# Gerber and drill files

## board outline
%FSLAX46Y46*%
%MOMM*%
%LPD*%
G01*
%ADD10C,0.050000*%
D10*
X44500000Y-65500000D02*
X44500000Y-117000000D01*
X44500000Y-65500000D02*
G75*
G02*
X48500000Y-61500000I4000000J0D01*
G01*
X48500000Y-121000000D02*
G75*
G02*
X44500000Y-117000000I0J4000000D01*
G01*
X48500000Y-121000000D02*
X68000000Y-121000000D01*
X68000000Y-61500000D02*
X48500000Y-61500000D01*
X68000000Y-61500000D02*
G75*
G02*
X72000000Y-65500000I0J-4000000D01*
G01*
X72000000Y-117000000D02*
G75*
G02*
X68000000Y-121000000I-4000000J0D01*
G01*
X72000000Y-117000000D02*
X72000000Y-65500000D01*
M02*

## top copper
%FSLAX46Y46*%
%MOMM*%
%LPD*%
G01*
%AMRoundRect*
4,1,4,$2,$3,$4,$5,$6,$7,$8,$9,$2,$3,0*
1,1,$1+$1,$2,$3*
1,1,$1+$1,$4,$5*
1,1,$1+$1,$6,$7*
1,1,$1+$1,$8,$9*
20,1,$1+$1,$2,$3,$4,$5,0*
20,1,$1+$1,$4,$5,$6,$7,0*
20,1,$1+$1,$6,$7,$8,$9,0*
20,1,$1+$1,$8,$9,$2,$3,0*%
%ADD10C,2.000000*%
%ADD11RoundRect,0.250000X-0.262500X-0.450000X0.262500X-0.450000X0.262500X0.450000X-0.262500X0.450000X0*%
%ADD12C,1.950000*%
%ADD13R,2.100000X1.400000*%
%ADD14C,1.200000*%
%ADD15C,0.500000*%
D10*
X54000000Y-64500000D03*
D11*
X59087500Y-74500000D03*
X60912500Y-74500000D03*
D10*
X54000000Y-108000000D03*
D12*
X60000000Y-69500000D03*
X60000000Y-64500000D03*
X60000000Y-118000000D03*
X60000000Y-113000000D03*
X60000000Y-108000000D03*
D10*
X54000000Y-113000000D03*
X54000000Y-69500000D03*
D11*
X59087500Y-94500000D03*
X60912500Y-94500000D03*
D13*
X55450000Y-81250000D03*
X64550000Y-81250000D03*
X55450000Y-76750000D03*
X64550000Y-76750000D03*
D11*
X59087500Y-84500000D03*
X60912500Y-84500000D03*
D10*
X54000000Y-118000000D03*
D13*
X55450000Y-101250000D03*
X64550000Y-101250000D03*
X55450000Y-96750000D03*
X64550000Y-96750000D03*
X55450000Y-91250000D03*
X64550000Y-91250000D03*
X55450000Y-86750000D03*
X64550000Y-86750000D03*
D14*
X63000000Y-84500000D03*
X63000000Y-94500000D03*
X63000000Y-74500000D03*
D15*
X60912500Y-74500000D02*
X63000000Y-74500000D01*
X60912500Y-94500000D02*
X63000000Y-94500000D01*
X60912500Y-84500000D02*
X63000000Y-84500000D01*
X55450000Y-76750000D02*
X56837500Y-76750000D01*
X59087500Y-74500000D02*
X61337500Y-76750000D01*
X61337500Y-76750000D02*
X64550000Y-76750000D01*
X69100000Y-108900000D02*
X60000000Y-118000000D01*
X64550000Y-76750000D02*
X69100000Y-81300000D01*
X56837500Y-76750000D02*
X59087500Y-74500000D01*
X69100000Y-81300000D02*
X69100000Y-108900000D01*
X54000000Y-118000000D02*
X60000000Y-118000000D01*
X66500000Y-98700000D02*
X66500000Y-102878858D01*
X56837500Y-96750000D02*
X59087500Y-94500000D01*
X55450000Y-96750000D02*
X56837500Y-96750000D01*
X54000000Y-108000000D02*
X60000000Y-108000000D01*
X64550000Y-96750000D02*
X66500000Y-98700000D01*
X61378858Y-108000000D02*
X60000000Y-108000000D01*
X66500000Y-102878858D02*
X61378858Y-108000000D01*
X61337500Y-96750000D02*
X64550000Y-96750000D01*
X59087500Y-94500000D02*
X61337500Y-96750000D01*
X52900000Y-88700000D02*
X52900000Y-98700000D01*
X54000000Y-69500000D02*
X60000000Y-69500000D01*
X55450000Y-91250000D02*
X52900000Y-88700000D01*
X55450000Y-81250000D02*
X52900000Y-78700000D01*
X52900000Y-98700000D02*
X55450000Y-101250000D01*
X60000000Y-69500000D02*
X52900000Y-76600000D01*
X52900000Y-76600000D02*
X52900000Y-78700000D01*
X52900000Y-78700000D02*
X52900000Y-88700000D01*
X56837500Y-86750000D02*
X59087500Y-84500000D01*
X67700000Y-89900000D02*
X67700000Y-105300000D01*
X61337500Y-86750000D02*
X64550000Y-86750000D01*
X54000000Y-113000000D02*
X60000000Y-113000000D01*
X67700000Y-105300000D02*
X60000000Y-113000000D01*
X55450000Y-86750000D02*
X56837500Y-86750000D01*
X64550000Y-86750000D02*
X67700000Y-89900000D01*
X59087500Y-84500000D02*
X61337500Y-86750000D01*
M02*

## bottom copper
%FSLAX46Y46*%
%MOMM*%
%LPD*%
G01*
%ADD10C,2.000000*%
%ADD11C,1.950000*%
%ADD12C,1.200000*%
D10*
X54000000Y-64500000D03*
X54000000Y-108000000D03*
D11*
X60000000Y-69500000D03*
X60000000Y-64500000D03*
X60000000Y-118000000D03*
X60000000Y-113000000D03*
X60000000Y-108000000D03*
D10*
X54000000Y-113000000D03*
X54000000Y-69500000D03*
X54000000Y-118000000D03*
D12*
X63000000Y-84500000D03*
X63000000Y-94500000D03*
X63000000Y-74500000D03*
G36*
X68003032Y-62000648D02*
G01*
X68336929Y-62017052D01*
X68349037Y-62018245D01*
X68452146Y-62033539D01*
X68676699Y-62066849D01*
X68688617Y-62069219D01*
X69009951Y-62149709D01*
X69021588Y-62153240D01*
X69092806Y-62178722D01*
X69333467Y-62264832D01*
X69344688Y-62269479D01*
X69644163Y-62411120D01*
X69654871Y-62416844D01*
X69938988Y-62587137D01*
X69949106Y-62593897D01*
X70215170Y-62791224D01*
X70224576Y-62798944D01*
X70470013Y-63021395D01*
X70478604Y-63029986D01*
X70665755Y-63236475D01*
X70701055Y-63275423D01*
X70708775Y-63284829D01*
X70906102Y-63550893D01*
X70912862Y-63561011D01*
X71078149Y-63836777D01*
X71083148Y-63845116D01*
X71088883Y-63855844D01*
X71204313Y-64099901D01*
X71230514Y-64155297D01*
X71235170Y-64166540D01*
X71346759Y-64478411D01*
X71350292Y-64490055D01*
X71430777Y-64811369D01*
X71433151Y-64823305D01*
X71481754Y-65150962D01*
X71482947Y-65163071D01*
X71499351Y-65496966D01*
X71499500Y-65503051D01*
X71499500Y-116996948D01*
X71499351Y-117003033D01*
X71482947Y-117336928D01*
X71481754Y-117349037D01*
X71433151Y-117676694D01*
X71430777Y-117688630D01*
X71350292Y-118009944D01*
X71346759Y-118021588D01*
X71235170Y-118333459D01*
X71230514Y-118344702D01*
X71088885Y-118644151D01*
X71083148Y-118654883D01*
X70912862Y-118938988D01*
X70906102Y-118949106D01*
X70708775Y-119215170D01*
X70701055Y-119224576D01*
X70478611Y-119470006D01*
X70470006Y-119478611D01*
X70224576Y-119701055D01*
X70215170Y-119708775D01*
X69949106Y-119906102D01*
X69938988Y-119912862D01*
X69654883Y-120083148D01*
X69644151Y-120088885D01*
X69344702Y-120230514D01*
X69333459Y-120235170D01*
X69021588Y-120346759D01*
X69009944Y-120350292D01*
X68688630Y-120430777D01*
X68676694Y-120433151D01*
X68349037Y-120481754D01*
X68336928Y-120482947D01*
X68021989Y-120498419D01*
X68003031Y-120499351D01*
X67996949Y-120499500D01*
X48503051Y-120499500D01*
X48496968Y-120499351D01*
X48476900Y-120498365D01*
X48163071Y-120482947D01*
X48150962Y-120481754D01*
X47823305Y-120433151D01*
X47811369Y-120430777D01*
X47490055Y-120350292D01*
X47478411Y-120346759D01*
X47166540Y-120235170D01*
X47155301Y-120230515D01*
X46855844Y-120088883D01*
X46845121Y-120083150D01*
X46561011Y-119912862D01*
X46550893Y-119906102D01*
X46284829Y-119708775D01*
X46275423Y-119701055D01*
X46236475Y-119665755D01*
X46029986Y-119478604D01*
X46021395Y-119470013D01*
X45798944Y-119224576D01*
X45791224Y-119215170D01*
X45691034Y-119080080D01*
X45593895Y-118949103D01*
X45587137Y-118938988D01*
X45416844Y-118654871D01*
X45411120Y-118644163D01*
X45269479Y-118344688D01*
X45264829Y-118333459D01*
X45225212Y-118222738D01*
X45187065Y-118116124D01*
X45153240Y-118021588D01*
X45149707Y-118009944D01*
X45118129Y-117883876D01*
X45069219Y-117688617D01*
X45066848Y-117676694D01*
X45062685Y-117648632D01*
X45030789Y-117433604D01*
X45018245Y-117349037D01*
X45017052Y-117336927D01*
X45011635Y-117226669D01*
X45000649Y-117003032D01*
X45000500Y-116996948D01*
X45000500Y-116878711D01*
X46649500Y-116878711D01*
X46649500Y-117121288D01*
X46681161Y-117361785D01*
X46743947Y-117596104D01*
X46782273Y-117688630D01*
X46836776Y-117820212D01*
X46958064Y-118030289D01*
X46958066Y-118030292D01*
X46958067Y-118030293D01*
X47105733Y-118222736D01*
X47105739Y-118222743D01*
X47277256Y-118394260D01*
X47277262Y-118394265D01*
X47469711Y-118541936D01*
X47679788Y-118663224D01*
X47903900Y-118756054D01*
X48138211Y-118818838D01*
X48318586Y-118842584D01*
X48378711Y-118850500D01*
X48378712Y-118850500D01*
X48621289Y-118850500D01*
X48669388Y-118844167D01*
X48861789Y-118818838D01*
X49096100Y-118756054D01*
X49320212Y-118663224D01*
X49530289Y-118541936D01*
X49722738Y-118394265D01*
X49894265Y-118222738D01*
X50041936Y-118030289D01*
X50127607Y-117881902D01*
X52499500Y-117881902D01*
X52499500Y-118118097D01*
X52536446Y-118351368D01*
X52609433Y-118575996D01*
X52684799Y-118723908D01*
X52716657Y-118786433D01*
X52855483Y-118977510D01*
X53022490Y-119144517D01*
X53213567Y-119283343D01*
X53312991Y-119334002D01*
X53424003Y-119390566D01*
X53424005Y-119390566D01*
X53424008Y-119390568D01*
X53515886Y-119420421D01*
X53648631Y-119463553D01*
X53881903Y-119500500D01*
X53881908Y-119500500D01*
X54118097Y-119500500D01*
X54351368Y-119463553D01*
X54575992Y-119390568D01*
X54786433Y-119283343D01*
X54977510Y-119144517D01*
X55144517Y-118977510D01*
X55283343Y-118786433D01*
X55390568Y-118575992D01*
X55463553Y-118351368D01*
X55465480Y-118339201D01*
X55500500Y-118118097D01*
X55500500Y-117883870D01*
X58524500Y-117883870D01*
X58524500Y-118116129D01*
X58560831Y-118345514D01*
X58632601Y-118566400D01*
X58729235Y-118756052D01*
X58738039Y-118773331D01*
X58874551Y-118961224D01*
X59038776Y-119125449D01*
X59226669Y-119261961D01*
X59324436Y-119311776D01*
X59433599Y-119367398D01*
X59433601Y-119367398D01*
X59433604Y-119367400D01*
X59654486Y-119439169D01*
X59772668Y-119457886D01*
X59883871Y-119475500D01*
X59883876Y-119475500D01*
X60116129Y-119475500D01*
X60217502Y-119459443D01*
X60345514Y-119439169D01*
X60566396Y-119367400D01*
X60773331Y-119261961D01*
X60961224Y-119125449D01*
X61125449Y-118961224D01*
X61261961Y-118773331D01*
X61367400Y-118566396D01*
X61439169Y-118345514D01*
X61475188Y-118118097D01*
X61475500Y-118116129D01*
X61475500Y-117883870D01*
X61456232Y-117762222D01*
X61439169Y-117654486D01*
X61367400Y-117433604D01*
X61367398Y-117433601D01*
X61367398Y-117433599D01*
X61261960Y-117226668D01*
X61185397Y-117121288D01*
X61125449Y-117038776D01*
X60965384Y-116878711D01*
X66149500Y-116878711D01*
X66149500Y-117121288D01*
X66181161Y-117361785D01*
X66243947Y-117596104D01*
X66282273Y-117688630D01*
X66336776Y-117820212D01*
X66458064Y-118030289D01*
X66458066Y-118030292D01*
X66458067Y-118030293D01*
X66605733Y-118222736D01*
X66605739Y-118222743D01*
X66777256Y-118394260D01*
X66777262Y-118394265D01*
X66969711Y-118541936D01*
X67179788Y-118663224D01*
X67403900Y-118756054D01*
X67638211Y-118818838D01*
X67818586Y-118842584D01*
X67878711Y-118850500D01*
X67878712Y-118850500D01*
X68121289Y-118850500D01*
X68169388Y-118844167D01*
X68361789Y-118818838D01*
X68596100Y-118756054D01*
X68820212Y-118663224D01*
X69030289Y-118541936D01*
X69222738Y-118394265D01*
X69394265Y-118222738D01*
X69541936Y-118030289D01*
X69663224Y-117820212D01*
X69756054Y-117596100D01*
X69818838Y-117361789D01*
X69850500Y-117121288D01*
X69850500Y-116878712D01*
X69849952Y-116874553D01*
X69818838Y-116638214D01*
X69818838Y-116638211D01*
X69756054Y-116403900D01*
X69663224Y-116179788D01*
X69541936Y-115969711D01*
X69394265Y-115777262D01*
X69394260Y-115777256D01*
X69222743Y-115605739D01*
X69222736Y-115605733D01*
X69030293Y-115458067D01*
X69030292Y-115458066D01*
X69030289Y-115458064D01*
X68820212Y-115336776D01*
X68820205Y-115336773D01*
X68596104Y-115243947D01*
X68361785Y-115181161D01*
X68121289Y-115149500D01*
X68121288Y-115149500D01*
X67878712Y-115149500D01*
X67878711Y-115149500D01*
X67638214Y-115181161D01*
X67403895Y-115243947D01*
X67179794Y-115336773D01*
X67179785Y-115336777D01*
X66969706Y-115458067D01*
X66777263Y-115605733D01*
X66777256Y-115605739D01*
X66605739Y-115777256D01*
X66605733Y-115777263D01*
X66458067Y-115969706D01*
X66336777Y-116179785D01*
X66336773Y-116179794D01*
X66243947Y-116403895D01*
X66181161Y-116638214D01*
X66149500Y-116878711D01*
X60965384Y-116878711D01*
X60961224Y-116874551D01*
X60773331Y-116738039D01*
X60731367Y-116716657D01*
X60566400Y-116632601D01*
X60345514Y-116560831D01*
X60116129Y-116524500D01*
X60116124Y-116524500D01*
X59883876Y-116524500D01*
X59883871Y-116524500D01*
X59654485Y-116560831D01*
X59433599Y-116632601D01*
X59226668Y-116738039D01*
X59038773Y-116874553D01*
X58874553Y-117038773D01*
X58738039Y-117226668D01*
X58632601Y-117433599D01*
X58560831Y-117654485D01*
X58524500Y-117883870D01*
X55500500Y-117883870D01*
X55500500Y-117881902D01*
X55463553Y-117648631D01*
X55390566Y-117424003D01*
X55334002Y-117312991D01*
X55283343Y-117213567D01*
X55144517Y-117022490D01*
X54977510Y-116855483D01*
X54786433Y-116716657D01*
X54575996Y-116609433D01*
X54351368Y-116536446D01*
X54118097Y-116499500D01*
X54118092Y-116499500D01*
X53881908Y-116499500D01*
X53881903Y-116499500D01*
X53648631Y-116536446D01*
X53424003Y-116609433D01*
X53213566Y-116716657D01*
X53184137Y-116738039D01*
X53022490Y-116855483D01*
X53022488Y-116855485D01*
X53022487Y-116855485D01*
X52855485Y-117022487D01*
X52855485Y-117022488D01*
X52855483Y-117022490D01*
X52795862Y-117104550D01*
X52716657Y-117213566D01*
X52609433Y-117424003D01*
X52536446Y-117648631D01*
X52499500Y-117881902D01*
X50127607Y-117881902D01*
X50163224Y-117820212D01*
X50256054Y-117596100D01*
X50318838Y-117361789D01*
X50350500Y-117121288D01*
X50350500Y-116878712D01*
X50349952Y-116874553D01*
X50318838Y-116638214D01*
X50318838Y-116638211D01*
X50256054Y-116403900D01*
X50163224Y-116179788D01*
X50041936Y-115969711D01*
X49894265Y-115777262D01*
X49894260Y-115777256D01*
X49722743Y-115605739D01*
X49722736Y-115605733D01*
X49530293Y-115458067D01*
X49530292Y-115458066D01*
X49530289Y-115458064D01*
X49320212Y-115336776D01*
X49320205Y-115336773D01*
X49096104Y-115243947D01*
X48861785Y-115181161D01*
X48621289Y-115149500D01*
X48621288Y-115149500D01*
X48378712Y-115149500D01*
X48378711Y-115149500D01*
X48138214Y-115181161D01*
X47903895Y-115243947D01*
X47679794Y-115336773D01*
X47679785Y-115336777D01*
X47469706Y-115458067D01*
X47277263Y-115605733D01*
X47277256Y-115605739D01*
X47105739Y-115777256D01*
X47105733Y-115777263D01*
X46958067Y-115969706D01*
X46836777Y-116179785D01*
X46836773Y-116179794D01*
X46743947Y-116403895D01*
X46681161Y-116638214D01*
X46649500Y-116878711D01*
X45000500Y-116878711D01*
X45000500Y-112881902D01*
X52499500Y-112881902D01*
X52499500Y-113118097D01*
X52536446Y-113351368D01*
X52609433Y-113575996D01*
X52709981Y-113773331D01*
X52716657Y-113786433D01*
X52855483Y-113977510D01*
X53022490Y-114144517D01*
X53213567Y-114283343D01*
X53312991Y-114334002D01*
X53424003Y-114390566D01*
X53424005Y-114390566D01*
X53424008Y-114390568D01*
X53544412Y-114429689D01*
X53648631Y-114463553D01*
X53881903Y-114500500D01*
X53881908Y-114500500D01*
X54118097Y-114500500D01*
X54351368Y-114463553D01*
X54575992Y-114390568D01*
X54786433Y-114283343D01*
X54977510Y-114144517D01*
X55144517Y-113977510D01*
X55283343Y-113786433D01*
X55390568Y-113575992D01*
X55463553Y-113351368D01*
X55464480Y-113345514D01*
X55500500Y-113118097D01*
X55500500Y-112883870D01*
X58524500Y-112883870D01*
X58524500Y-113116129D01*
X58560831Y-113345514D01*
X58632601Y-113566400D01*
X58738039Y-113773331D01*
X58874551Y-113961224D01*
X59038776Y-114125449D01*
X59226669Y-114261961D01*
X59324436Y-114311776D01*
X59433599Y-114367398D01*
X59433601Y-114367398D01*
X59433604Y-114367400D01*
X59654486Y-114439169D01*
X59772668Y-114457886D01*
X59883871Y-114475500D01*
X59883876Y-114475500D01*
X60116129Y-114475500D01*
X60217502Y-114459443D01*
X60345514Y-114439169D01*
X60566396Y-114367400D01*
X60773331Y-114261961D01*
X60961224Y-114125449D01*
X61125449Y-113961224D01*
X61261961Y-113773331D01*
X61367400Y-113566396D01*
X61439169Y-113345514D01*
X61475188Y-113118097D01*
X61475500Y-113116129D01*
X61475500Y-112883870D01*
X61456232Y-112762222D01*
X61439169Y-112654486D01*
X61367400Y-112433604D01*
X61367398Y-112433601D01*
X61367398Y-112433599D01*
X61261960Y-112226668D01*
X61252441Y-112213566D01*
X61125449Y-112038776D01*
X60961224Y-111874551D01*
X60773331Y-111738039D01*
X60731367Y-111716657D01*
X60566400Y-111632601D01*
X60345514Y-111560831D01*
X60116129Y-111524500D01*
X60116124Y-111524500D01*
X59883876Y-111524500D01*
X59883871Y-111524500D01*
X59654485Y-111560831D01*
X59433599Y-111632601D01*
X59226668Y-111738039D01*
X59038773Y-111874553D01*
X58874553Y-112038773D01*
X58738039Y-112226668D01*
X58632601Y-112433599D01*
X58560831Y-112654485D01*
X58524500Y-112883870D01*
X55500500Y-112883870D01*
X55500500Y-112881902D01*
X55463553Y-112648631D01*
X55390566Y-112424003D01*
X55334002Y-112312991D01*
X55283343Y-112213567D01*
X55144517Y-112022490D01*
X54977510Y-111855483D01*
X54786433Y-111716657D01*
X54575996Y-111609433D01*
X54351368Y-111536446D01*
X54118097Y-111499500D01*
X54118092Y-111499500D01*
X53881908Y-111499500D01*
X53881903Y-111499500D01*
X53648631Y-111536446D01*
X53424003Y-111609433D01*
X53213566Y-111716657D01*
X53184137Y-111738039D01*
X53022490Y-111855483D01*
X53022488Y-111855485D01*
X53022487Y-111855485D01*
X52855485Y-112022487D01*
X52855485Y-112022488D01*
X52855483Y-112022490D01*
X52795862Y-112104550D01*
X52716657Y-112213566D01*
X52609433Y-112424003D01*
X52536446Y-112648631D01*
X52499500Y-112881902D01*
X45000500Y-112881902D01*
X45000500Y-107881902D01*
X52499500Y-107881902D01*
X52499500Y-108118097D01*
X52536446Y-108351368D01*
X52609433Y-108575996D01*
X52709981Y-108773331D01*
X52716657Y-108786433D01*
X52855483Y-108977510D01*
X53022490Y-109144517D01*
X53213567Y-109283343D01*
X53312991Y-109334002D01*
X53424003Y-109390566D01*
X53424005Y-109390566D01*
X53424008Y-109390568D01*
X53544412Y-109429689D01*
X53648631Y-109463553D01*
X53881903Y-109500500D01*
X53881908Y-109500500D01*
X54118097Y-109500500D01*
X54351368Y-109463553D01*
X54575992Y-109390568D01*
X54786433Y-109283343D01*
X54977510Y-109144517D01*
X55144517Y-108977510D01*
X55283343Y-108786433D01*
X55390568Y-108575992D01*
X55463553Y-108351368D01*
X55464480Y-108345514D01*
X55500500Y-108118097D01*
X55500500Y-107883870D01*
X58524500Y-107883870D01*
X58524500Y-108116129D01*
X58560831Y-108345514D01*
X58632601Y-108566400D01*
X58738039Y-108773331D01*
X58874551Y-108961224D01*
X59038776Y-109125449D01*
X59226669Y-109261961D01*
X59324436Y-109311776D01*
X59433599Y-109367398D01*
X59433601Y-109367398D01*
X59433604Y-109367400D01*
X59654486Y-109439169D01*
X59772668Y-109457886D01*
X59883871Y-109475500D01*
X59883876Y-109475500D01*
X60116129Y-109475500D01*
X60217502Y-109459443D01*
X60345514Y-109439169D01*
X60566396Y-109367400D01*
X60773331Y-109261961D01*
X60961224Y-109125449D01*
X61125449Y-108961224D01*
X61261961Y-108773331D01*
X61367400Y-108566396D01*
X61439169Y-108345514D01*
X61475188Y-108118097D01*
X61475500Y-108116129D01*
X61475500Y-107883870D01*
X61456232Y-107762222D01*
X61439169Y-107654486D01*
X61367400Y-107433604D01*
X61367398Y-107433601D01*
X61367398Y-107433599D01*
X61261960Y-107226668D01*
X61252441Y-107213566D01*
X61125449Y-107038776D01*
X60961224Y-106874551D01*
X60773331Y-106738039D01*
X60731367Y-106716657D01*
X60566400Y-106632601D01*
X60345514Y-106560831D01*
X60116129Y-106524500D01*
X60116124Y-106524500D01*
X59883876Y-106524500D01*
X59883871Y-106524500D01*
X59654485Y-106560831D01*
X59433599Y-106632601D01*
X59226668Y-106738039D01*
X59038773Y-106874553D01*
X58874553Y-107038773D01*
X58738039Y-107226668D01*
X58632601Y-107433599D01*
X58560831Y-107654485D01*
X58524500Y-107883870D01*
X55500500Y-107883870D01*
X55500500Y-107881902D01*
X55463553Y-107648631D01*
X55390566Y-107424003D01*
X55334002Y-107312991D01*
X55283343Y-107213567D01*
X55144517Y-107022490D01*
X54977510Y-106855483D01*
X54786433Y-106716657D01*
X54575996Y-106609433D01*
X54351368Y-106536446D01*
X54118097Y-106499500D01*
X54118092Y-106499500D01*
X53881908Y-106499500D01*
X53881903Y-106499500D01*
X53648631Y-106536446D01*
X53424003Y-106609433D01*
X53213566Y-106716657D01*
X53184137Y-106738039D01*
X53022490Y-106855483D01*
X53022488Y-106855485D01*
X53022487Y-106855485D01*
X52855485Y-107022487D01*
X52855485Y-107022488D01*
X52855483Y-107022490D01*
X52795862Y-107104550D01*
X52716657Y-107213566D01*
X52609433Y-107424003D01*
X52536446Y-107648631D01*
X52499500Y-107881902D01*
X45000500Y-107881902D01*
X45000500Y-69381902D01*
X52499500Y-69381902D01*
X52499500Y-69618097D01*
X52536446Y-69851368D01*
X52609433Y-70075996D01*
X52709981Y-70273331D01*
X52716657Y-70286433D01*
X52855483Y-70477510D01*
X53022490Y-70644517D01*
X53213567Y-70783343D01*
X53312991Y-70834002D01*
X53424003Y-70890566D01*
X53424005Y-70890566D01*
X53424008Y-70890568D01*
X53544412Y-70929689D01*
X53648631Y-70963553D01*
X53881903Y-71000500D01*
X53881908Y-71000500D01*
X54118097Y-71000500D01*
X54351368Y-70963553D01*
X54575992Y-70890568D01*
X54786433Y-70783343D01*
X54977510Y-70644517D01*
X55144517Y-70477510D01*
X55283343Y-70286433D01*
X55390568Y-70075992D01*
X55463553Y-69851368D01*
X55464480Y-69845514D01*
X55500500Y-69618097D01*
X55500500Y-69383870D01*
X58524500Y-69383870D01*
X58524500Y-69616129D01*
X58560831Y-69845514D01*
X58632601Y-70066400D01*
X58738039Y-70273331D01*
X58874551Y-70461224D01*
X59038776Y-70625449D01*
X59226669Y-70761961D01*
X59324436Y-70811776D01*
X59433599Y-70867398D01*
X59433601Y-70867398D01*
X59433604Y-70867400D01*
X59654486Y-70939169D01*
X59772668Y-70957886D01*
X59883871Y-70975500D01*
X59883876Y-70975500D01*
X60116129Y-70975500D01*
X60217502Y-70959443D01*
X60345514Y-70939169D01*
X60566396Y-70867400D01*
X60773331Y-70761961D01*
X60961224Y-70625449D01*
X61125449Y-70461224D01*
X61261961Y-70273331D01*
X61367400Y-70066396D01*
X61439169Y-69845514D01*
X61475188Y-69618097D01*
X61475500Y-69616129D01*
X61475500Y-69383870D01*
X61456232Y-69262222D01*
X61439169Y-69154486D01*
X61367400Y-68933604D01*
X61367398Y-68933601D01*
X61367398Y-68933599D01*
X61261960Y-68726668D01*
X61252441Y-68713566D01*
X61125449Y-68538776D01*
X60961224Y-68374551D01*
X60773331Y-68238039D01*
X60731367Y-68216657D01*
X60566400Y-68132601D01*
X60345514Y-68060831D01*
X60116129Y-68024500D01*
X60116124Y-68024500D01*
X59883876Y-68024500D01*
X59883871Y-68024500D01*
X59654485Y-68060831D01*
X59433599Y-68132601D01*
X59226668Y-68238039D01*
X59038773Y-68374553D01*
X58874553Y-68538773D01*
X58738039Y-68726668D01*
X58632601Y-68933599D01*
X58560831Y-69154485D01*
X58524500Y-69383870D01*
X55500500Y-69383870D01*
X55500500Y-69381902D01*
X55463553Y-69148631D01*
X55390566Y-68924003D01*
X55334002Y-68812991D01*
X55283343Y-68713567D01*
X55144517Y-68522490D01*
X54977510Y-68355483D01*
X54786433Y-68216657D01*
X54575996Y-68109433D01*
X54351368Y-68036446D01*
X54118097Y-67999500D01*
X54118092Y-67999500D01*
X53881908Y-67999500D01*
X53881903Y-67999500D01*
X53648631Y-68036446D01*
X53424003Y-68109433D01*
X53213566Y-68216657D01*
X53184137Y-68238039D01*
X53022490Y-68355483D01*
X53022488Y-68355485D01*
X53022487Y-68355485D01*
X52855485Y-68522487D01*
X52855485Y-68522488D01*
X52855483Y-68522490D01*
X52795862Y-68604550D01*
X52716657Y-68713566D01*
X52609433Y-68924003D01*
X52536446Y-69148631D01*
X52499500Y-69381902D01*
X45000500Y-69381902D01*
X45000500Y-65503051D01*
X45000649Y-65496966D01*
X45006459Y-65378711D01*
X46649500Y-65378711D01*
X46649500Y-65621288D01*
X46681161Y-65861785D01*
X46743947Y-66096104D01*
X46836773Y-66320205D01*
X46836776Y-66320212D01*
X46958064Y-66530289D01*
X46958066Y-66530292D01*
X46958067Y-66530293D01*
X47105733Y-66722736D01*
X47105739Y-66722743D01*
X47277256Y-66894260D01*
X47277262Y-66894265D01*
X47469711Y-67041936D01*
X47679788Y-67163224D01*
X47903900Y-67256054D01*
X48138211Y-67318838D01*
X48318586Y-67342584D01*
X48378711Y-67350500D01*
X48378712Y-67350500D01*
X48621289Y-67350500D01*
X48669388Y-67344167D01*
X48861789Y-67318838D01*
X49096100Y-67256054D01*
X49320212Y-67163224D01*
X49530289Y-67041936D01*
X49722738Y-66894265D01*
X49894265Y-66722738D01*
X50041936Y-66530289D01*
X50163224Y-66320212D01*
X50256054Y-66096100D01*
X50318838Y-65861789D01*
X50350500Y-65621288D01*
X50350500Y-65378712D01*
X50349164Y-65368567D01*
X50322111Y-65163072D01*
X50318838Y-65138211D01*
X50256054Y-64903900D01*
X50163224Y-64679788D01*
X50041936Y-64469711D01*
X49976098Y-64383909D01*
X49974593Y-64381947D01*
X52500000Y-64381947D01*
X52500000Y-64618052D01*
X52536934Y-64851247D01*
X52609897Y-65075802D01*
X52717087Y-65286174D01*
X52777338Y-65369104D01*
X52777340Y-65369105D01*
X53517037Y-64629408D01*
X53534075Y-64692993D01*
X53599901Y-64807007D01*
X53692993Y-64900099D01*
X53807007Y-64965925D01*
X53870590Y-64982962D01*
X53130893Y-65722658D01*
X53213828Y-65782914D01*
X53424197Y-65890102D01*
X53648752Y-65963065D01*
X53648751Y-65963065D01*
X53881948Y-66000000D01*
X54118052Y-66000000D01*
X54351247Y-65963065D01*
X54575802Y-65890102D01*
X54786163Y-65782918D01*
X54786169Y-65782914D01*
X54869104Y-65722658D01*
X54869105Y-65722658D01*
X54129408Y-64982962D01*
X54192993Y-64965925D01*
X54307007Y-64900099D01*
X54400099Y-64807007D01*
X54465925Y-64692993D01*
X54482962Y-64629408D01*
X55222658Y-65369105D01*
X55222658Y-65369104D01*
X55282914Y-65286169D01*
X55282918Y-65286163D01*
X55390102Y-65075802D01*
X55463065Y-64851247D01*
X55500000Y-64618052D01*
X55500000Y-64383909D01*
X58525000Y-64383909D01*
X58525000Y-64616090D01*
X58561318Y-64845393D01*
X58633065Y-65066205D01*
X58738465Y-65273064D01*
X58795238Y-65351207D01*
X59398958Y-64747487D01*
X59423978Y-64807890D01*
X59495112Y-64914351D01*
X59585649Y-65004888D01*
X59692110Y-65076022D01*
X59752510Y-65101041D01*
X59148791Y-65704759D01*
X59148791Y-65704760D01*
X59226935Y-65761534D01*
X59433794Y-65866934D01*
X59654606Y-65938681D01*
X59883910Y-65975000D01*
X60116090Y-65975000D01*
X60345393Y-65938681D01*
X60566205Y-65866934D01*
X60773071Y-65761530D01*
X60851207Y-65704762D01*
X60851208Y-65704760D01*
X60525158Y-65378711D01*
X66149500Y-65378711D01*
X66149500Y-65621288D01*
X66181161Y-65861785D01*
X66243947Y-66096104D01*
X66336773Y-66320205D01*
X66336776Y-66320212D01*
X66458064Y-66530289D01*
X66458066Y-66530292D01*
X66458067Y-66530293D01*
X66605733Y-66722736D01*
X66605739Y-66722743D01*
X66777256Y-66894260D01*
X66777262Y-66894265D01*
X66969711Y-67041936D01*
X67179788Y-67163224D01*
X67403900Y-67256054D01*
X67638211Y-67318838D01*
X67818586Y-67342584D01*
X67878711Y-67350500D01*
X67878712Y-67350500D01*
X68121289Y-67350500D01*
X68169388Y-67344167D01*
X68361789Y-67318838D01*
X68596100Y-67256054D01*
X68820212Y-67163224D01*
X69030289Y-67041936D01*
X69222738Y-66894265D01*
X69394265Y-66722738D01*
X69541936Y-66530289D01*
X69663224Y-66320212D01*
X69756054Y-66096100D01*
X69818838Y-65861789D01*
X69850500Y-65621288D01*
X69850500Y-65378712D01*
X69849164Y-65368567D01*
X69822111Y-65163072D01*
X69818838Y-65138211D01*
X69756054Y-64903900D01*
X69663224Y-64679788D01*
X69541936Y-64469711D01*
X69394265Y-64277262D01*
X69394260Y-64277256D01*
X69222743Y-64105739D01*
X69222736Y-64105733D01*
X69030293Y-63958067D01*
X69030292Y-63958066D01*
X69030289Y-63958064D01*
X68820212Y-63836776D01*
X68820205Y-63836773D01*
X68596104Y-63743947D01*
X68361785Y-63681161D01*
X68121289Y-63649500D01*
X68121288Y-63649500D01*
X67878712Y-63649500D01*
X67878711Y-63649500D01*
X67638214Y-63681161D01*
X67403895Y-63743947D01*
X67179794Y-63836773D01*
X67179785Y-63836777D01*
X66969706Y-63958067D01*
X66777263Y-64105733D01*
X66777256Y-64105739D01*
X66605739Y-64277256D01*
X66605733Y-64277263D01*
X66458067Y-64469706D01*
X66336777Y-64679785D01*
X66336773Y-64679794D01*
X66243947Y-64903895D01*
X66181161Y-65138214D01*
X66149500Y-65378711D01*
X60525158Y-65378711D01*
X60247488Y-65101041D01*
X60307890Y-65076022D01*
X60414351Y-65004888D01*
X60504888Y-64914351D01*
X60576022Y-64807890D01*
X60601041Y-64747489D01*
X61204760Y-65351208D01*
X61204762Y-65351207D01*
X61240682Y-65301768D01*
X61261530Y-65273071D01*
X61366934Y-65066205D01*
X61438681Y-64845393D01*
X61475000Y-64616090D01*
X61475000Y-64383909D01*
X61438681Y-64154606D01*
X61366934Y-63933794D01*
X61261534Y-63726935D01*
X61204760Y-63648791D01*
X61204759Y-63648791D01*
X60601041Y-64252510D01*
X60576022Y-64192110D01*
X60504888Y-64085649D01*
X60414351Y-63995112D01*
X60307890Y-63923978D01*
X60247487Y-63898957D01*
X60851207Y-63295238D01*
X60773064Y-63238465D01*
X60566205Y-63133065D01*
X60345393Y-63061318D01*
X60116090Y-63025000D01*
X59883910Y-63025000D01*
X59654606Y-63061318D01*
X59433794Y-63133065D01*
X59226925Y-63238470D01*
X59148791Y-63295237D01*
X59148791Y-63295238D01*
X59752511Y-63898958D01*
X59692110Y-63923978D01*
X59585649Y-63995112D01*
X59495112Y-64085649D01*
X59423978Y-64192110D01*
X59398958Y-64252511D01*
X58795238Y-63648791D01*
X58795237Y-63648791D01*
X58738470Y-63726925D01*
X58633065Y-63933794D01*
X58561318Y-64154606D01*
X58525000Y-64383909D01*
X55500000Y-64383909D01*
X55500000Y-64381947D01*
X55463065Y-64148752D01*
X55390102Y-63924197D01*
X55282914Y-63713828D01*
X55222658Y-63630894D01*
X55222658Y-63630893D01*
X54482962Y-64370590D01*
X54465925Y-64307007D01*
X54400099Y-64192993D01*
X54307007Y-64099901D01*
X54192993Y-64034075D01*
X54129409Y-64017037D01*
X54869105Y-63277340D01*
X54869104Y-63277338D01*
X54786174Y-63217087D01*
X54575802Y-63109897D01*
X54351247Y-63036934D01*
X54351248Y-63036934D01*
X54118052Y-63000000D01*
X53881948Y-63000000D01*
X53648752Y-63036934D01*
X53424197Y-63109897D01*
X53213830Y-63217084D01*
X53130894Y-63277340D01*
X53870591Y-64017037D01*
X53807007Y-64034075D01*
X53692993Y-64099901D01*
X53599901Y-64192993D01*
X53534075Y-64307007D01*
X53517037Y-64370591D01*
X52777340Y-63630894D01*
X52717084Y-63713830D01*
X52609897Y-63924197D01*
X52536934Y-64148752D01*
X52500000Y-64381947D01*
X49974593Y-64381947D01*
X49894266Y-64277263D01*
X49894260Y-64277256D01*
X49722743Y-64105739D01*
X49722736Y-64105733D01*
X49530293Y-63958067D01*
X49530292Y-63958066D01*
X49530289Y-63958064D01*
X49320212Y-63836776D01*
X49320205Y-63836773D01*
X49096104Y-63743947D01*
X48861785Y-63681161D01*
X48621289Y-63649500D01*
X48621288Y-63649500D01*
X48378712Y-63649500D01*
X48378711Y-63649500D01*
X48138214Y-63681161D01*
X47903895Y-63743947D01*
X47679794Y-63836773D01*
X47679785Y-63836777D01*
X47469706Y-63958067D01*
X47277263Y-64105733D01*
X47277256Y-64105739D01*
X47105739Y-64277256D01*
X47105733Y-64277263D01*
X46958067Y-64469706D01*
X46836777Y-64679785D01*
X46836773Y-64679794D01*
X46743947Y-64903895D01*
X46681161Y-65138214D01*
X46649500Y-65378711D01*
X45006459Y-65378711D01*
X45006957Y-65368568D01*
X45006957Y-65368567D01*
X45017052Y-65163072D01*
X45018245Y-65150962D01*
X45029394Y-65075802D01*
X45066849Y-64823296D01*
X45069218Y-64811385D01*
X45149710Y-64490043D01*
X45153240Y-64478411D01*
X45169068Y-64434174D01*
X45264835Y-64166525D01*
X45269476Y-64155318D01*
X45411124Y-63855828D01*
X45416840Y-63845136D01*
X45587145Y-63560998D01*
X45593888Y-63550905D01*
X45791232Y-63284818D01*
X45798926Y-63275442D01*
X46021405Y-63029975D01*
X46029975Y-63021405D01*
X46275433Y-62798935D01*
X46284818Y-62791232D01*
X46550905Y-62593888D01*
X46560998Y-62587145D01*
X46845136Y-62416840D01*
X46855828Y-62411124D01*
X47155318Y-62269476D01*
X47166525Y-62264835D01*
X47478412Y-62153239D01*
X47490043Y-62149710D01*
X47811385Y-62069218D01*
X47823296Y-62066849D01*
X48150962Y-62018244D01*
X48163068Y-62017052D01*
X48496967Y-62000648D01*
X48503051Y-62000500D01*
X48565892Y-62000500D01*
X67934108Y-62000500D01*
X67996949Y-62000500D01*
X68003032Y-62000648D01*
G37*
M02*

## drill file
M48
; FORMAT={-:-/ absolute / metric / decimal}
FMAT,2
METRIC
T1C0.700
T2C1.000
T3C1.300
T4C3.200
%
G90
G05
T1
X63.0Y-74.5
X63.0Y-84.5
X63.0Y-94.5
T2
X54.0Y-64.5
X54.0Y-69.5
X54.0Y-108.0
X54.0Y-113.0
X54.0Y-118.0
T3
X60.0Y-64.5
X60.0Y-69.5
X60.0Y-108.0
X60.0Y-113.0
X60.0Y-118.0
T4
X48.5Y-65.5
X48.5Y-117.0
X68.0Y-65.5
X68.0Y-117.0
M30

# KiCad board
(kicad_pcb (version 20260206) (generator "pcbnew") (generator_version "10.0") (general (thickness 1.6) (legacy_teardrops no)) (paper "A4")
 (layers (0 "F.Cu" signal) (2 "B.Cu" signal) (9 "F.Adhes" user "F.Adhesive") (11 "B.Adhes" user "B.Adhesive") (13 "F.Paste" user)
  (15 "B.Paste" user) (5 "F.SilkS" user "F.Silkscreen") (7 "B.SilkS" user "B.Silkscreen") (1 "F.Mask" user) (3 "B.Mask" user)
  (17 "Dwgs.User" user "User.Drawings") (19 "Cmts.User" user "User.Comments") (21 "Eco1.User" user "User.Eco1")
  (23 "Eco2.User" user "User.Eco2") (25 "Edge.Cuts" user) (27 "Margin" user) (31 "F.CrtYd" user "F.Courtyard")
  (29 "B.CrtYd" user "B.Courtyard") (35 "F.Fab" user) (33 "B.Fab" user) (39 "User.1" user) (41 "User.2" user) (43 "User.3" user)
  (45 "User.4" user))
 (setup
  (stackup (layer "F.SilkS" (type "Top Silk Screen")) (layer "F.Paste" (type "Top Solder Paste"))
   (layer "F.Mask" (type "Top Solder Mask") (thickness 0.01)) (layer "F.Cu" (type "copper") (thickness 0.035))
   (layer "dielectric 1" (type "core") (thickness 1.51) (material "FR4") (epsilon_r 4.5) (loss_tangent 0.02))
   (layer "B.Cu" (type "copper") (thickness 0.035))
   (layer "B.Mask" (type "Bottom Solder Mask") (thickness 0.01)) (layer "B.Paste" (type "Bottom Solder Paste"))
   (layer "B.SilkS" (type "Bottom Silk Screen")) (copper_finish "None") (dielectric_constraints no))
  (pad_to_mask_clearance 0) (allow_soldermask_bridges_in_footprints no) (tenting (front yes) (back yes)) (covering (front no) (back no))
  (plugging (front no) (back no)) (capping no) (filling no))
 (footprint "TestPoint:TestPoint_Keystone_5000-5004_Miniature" (layer "F.Cu") (at 54 64.5)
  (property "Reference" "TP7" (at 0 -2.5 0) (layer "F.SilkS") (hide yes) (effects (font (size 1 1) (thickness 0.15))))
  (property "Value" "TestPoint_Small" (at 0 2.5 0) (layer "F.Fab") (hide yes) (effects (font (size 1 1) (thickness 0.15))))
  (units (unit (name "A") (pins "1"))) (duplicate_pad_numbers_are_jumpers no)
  (pad "1" thru_hole circle (at 0 0) (size 2 2) (drill 1) (layers "*.Cu" "*.Mask") (remove_unused_layers no) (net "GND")))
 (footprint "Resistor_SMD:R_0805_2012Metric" (layer "F.Cu") (at 60 74.5)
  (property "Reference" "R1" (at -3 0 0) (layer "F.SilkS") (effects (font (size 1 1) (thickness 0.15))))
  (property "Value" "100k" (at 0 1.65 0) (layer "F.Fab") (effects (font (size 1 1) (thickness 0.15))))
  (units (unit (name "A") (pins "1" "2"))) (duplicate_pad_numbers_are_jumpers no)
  (pad "1" smd roundrect (at -0.9125 0) (size 1.025 1.4) (layers "F.Cu" "F.Mask" "F.Paste") (roundrect_rratio 0.243902) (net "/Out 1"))
  (pad "2" smd roundrect (at 0.9125 0) (size 1.025 1.4) (layers "F.Cu" "F.Mask" "F.Paste") (roundrect_rratio 0.243902) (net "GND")))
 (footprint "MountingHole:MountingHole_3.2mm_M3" (layer "F.Cu") (at 68 117)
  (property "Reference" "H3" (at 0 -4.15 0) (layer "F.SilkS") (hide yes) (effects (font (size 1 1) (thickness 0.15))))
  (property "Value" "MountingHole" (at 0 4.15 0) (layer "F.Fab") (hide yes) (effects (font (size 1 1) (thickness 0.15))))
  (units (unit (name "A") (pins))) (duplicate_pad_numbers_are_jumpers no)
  (pad "" np_thru_hole circle (at 0 0) (size 3.2 3.2) (drill 3.2) (layers "*.Cu" "*.Mask")))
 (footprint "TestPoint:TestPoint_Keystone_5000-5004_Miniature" (layer "F.Cu") (at 54 108)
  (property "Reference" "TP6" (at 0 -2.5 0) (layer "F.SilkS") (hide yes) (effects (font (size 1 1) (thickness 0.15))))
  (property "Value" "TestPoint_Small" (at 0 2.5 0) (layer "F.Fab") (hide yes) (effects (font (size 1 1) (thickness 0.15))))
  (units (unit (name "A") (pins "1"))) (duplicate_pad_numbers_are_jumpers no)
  (pad "1" thru_hole circle (at 0 0) (size 2 2) (drill 1) (layers "*.Cu" "*.Mask") (remove_unused_layers no) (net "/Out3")))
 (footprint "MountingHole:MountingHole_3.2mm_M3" (layer "F.Cu") (at 48.5 117)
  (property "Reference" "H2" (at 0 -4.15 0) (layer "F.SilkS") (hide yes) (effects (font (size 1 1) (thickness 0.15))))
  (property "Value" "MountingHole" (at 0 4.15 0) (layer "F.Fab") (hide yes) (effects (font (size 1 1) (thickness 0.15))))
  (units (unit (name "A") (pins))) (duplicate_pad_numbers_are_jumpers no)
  (pad "" np_thru_hole circle (at 0 0) (size 3.2 3.2) (drill 3.2) (layers "*.Cu" "*.Mask")))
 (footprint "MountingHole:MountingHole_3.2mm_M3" (layer "F.Cu") (at 68 65.5)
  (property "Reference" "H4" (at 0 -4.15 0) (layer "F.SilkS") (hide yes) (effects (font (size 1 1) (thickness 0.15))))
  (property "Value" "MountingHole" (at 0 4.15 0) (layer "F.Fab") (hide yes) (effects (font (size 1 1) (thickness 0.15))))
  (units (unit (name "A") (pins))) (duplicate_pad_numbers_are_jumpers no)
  (pad "" np_thru_hole circle (at 0 0) (size 3.2 3.2) (drill 3.2) (layers "*.Cu" "*.Mask")))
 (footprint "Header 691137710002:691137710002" (layer "F.Cu") (at 60 67 90)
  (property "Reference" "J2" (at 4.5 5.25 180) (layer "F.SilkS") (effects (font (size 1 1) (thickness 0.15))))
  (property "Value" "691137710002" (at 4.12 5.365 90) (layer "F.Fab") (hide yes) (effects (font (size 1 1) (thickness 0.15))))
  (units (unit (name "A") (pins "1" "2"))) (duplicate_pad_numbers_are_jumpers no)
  (pad "1" thru_hole circle (at -2.5 0 90) (size 1.95 1.95) (drill 1.3) (layers "*.Cu" "*.Mask") (remove_unused_layers no) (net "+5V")
   (solder_mask_margin 0.102))
  (pad "2" thru_hole circle (at 2.5 0 90) (size 1.95 1.95) (drill 1.3) (layers "*.Cu" "*.Mask") (remove_unused_layers no) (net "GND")
   (solder_mask_margin 0.102)))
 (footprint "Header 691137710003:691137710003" (layer "F.Cu") (at 60 113 90)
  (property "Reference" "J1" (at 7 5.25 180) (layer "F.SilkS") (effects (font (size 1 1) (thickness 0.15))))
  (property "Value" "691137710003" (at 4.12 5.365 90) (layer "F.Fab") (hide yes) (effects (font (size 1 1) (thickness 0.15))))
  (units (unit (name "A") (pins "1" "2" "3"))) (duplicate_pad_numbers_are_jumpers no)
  (pad "1" thru_hole circle (at -5 0 90) (size 1.95 1.95) (drill 1.3) (layers "*.Cu" "*.Mask") (remove_unused_layers no) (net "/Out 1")
   (solder_mask_margin 0.102))
  (pad "2" thru_hole circle (at 0 0 90) (size 1.95 1.95) (drill 1.3) (layers "*.Cu" "*.Mask") (remove_unused_layers no) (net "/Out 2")
   (solder_mask_margin 0.102))
  (pad "3" thru_hole circle (at 5 0 90) (size 1.95 1.95) (drill 1.3) (layers "*.Cu" "*.Mask") (remove_unused_layers no) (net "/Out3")
   (solder_mask_margin 0.102)))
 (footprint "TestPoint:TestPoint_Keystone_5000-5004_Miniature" (layer "F.Cu") (at 54 113)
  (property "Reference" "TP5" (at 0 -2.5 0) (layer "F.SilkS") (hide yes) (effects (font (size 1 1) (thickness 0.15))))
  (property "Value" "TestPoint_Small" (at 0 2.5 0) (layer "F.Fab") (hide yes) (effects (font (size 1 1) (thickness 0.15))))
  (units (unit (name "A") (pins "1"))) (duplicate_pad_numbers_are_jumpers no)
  (pad "1" thru_hole circle (at 0 0) (size 2 2) (drill 1) (layers "*.Cu" "*.Mask") (remove_unused_layers no) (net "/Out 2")))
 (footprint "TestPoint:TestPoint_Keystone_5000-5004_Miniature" (layer "F.Cu") (at 54 69.5)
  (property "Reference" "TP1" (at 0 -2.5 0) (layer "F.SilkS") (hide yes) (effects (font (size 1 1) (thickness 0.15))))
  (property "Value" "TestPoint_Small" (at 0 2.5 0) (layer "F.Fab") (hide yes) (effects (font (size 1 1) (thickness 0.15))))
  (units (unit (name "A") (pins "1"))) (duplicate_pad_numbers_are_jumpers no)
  (pad "1" thru_hole circle (at 0 0) (size 2 2) (drill 1) (layers "*.Cu" "*.Mask") (remove_unused_layers no) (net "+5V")))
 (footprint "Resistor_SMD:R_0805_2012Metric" (layer "F.Cu") (at 60 94.5)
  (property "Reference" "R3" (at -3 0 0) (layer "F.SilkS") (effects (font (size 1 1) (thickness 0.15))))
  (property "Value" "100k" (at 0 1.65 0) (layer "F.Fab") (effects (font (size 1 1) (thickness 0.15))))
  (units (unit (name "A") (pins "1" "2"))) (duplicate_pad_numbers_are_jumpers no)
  (pad "1" smd roundrect (at -0.9125 0) (size 1.025 1.4) (layers "F.Cu" "F.Mask" "F.Paste") (roundrect_rratio 0.243902) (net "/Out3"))
  (pad "2" smd roundrect (at 0.9125 0) (size 1.025 1.4) (layers "F.Cu" "F.Mask" "F.Paste") (roundrect_rratio 0.243902) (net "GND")))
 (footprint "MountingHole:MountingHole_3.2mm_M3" (layer "F.Cu") (at 48.5 65.5)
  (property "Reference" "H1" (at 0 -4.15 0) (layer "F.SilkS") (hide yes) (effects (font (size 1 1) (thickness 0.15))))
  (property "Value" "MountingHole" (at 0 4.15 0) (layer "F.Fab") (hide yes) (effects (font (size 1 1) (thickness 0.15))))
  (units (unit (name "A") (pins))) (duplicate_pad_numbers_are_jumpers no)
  (pad "" np_thru_hole circle (at 0 0) (size 3.2 3.2) (drill 3.2) (layers "*.Cu" "*.Mask")))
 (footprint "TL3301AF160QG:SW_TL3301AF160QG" (layer "F.Cu") (at 60 79)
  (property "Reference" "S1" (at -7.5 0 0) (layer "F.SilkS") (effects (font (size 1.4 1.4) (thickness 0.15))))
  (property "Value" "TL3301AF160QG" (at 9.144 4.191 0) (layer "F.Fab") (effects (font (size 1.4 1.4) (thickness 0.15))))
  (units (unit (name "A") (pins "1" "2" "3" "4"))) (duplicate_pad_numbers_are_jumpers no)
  (pad "1" smd rect (at -4.55 2.25) (size 2.1 1.4) (layers "F.Cu" "F.Mask" "F.Paste") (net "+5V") (solder_mask_margin 0.102))
  (pad "2" smd rect (at 4.55 2.25) (size 2.1 1.4) (layers "F.Cu" "F.Mask" "F.Paste") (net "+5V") (solder_mask_margin 0.102))
  (pad "3" smd rect (at -4.55 -2.25) (size 2.1 1.4) (layers "F.Cu" "F.Mask" "F.Paste") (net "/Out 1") (solder_mask_margin 0.102))
  (pad "4" smd rect (at 4.55 -2.25) (size 2.1 1.4) (layers "F.Cu" "F.Mask" "F.Paste") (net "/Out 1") (solder_mask_margin 0.102)))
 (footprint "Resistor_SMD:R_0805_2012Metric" (layer "F.Cu") (at 60 84.5)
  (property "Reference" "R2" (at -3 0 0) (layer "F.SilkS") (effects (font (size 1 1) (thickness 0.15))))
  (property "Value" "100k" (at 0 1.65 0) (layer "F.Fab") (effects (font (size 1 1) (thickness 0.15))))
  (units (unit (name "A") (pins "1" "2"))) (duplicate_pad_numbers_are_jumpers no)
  (pad "1" smd roundrect (at -0.9125 0) (size 1.025 1.4) (layers "F.Cu" "F.Mask" "F.Paste") (roundrect_rratio 0.243902) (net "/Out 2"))
  (pad "2" smd roundrect (at 0.9125 0) (size 1.025 1.4) (layers "F.Cu" "F.Mask" "F.Paste") (roundrect_rratio 0.243902) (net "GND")))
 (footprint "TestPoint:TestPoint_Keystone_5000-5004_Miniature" (layer "F.Cu") (at 54 118)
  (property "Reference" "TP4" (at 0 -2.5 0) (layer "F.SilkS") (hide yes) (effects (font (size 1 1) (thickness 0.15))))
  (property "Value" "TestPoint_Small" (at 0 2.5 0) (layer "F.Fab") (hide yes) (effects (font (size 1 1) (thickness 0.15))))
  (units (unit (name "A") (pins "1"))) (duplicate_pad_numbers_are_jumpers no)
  (pad "1" thru_hole circle (at 0 0) (size 2 2) (drill 1) (layers "*.Cu" "*.Mask") (remove_unused_layers no) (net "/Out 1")))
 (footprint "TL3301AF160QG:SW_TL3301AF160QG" (layer "F.Cu") (at 60 99)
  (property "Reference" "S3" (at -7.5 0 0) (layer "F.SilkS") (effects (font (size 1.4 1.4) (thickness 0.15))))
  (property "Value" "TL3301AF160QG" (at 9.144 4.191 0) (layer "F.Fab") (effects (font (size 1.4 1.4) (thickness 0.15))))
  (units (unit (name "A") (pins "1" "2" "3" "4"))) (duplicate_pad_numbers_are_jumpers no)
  (pad "1" smd rect (at -4.55 2.25) (size 2.1 1.4) (layers "F.Cu" "F.Mask" "F.Paste") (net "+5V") (solder_mask_margin 0.102))
  (pad "2" smd rect (at 4.55 2.25) (size 2.1 1.4) (layers "F.Cu" "F.Mask" "F.Paste") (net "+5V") (solder_mask_margin 0.102))
  (pad "3" smd rect (at -4.55 -2.25) (size 2.1 1.4) (layers "F.Cu" "F.Mask" "F.Paste") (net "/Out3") (solder_mask_margin 0.102))
  (pad "4" smd rect (at 4.55 -2.25) (size 2.1 1.4) (layers "F.Cu" "F.Mask" "F.Paste") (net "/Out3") (solder_mask_margin 0.102)))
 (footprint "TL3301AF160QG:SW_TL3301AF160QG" (layer "F.Cu") (at 60 89)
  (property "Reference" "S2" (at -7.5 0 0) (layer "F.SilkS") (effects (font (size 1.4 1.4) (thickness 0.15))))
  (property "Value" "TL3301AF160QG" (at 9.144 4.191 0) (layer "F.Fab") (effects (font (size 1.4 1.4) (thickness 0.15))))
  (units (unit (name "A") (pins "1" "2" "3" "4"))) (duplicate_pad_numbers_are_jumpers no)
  (pad "1" smd rect (at -4.55 2.25) (size 2.1 1.4) (layers "F.Cu" "F.Mask" "F.Paste") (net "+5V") (solder_mask_margin 0.102))
  (pad "2" smd rect (at 4.55 2.25) (size 2.1 1.4) (layers "F.Cu" "F.Mask" "F.Paste") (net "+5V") (solder_mask_margin 0.102))
  (pad "3" smd rect (at -4.55 -2.25) (size 2.1 1.4) (layers "F.Cu" "F.Mask" "F.Paste") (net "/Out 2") (solder_mask_margin 0.102))
  (pad "4" smd rect (at 4.55 -2.25) (size 2.1 1.4) (layers "F.Cu" "F.Mask" "F.Paste") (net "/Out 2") (solder_mask_margin 0.102)))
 (gr_line (start 44.5 65.5) (end 44.5 117) (stroke (width 0.05) (type default)) (layer "Edge.Cuts"))
 (gr_arc (start 44.5 65.5) (mid 45.671573 62.671573) (end 48.5 61.5) (stroke (width 0.05) (type default)) (layer "Edge.Cuts"))
 (gr_arc (start 48.5 121) (mid 45.671573 119.828427) (end 44.5 117) (stroke (width 0.05) (type default)) (layer "Edge.Cuts"))
 (gr_line (start 48.5 121) (end 68 121) (stroke (width 0.05) (type default)) (layer "Edge.Cuts"))
 (gr_line (start 68 61.5) (end 48.5 61.5) (stroke (width 0.05) (type default)) (layer "Edge.Cuts"))
 (gr_arc (start 68 61.5) (mid 70.828427 62.671573) (end 72 65.5) (stroke (width 0.05) (type default)) (layer "Edge.Cuts"))
 (gr_arc (start 72 117) (mid 70.828427 119.828427) (end 68 121) (stroke (width 0.05) (type default)) (layer "Edge.Cuts"))
 (gr_line (start 72 117) (end 72 65.5) (stroke (width 0.05) (type default)) (layer "Edge.Cuts"))
 (segment (start 60.9125 74.5) (end 63 74.5) (width 0.5) (layer "F.Cu") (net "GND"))
 (segment (start 60.9125 94.5) (end 63 94.5) (width 0.5) (layer "F.Cu") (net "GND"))
 (segment (start 60.9125 84.5) (end 63 84.5) (width 0.5) (layer "F.Cu") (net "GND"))
 (via (at 63 84.5) (size 1.2) (drill 0.7) (layers "F.Cu" "B.Cu") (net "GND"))
 (via (at 63 94.5) (size 1.2) (drill 0.7) (layers "F.Cu" "B.Cu") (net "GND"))
 (via (at 63 74.5) (size 1.2) (drill 0.7) (layers "F.Cu" "B.Cu") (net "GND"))
 (segment (start 55.45 76.75) (end 56.8375 76.75) (width 0.5) (layer "F.Cu") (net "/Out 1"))
 (segment (start 59.0875 74.5) (end 61.3375 76.75) (width 0.5) (layer "F.Cu") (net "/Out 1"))
 (segment (start 61.3375 76.75) (end 64.55 76.75) (width 0.5) (layer "F.Cu") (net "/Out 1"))
 (segment (start 69.1 108.9) (end 60 118) (width 0.5) (layer "F.Cu") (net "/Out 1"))
 (segment (start 64.55 76.75) (end 69.1 81.3) (width 0.5) (layer "F.Cu") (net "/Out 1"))
 (segment (start 56.8375 76.75) (end 59.0875 74.5) (width 0.5) (layer "F.Cu") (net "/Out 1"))
 (segment (start 69.1 81.3) (end 69.1 108.9) (width 0.5) (layer "F.Cu") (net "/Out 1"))
 (segment (start 54 118) (end 60 118) (width 0.5) (layer "F.Cu") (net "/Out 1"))
 (segment (start 66.5 98.7) (end 66.5 102.878858) (width 0.5) (layer "F.Cu") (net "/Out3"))
 (segment (start 56.8375 96.75) (end 59.0875 94.5) (width 0.5) (layer "F.Cu") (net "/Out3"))
 (segment (start 55.45 96.75) (end 56.8375 96.75) (width 0.5) (layer "F.Cu") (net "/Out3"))
 (segment (start 54 108) (end 60 108) (width 0.5) (layer "F.Cu") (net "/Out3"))
 (segment (start 64.55 96.75) (end 66.5 98.7) (width 0.5) (layer "F.Cu") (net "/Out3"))
 (segment (start 61.378858 108) (end 60 108) (width 0.5) (layer "F.Cu") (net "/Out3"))
 (segment (start 66.5 102.878858) (end 61.378858 108) (width 0.5) (layer "F.Cu") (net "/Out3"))
 (segment (start 61.3375 96.75) (end 64.55 96.75) (width 0.5) (layer "F.Cu") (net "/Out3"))
 (segment (start 59.0875 94.5) (end 61.3375 96.75) (width 0.5) (layer "F.Cu") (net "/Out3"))
 (segment (start 52.9 88.7) (end 52.9 98.7) (width 0.5) (layer "F.Cu") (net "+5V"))
 (segment (start 54 69.5) (end 60 69.5) (width 0.5) (layer "F.Cu") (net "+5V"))
 (segment (start 55.45 91.25) (end 52.9 88.7) (width 0.5) (layer "F.Cu") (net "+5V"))
 (segment (start 55.45 81.25) (end 52.9 78.7) (width 0.5) (layer "F.Cu") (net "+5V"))
 (segment (start 52.9 98.7) (end 55.45 101.25) (width 0.5) (layer "F.Cu") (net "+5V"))
 (segment (start 60 69.5) (end 52.9 76.6) (width 0.5) (layer "F.Cu") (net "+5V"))
 (segment (start 52.9 76.6) (end 52.9 78.7) (width 0.5) (layer "F.Cu") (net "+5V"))
 (segment (start 52.9 78.7) (end 52.9 88.7) (width 0.5) (layer "F.Cu") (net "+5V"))
 (segment (start 56.8375 86.75) (end 59.0875 84.5) (width 0.5) (layer "F.Cu") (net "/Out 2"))
 (segment (start 67.7 89.9) (end 67.7 105.3) (width 0.5) (layer "F.Cu") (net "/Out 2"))
 (segment (start 61.3375 86.75) (end 64.55 86.75) (width 0.5) (layer "F.Cu") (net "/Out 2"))
 (segment (start 54 113) (end 60 113) (width 0.5) (layer "F.Cu") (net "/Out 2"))
 (segment (start 67.7 105.3) (end 60 113) (width 0.5) (layer "F.Cu") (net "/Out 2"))
 (segment (start 55.45 86.75) (end 56.8375 86.75) (width 0.5) (layer "F.Cu") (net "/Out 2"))
 (segment (start 64.55 86.75) (end 67.7 89.9) (width 0.5) (layer "F.Cu") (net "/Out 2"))
 (segment (start 59.0875 84.5) (end 61.3375 86.75) (width 0.5) (layer "F.Cu") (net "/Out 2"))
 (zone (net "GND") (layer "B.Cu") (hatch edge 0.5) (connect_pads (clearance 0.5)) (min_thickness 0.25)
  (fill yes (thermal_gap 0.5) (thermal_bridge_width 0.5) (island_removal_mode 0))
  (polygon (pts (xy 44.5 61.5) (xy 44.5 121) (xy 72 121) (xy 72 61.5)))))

